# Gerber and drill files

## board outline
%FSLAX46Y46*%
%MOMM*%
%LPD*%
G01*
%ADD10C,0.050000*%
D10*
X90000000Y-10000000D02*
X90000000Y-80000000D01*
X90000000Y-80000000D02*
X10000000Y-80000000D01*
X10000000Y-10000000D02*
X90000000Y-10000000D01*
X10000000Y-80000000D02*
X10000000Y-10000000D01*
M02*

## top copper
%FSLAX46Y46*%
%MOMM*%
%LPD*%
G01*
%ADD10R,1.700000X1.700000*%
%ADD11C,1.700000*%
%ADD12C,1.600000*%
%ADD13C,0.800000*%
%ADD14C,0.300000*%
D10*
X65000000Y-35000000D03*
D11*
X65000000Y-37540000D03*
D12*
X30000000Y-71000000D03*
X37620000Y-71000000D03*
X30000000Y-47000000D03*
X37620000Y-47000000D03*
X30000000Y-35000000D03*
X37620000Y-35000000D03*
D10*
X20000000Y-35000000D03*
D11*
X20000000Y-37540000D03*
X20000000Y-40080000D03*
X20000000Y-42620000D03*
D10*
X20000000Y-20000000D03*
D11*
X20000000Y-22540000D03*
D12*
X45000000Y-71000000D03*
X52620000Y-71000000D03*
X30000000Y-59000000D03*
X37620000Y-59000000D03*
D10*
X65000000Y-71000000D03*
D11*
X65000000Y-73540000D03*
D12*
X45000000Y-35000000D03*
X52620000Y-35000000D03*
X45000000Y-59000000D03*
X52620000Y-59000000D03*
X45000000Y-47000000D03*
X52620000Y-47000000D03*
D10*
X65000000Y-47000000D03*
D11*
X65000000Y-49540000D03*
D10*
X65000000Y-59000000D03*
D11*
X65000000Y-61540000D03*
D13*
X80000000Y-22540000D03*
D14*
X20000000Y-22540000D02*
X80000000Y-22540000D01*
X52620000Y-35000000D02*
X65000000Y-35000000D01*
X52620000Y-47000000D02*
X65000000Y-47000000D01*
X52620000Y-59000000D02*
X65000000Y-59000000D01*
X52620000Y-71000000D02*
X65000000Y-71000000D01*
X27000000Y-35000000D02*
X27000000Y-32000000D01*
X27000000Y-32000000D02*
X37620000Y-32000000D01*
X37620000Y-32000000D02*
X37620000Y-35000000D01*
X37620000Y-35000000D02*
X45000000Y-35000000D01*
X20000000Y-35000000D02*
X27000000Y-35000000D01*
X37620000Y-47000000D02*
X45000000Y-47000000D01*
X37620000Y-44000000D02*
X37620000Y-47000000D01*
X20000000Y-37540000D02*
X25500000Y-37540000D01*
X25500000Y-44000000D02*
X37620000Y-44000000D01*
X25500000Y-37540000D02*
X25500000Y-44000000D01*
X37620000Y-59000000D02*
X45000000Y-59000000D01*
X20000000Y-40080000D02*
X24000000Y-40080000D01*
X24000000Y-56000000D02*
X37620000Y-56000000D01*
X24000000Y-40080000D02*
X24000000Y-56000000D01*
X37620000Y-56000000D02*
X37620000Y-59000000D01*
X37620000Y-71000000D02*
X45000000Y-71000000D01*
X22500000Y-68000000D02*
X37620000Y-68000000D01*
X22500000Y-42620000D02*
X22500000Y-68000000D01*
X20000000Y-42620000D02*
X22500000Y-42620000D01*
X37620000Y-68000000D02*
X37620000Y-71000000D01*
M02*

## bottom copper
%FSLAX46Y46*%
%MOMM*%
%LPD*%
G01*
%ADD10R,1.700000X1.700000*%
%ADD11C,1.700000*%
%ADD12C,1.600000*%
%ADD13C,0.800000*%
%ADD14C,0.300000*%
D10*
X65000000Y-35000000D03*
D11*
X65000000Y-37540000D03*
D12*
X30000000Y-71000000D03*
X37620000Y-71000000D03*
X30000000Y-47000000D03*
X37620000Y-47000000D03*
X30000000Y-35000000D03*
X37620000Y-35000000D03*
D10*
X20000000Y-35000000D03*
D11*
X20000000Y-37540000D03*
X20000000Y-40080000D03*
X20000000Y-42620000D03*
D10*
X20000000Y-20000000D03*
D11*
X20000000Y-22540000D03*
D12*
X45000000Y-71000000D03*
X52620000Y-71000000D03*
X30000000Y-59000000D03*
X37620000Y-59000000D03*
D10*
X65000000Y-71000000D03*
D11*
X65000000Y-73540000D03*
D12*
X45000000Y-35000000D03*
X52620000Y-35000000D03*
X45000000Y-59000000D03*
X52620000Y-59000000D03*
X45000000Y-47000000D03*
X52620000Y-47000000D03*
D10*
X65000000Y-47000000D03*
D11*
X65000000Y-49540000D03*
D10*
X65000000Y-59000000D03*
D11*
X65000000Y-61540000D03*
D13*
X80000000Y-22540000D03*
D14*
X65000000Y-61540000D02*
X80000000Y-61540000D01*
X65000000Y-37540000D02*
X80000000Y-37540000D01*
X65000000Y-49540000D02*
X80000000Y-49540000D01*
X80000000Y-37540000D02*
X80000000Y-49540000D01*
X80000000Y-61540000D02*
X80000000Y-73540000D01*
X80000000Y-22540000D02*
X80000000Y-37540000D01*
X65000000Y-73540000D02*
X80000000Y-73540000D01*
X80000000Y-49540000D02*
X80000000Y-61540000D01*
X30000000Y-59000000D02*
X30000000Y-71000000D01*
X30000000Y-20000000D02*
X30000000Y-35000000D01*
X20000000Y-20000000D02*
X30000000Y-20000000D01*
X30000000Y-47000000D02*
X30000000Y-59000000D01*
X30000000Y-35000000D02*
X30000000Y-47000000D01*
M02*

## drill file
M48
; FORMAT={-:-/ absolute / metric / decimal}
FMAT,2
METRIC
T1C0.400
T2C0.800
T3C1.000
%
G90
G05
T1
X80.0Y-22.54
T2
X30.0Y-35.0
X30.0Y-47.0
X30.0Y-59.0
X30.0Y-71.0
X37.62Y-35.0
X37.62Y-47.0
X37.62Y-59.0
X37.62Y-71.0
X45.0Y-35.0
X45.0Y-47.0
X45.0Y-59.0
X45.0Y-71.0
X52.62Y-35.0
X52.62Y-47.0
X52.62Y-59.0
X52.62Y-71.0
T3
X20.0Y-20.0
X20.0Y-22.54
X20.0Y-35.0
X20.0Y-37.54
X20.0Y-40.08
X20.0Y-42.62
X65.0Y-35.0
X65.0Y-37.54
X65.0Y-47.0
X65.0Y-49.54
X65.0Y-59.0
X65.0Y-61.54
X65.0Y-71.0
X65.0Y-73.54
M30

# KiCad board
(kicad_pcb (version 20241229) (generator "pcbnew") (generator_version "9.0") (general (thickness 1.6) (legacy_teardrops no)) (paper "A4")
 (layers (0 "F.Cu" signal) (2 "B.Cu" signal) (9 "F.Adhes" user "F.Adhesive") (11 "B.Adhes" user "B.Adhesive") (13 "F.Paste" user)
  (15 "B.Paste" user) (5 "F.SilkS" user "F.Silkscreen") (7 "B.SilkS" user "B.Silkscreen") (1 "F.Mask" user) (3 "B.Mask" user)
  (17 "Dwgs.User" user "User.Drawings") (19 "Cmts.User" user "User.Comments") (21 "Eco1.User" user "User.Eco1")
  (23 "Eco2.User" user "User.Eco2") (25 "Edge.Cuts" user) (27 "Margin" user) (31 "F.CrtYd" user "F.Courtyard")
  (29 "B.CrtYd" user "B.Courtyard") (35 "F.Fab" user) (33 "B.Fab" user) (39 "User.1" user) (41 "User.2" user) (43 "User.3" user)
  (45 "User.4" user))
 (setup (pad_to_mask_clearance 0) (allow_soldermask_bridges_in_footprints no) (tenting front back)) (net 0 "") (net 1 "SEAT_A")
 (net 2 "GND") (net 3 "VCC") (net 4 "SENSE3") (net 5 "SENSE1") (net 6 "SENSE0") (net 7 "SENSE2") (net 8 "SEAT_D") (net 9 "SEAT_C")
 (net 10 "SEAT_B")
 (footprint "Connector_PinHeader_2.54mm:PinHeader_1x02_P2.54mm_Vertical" (layer "F.Cu") (at 65 35)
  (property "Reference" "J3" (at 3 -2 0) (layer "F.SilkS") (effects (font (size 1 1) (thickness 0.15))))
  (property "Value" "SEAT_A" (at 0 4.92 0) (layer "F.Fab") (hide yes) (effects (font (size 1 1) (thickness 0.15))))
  (pad "1" thru_hole rect (at 0 0) (size 1.7 1.7) (drill 1) (layers "*.Cu" "*.Mask") (remove_unused_layers no) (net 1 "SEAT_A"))
  (pad "2" thru_hole circle (at 0 2.54) (size 1.7 1.7) (drill 1) (layers "*.Cu" "*.Mask") (remove_unused_layers no) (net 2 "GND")))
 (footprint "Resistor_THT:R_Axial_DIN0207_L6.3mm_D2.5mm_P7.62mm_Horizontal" (layer "F.Cu") (at 30 71)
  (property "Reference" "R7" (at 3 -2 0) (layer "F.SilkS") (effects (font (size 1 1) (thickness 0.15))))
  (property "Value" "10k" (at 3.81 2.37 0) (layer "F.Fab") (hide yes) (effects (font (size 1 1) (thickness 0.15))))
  (pad "1" thru_hole circle (at 0 0) (size 1.6 1.6) (drill 0.8) (layers "*.Cu" "*.Mask") (remove_unused_layers no) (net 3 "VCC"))
  (pad "2" thru_hole circle (at 7.62 0) (size 1.6 1.6) (drill 0.8) (layers "*.Cu" "*.Mask") (remove_unused_layers no) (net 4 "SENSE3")))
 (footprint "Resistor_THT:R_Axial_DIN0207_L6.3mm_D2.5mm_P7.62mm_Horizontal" (layer "F.Cu") (at 30 47)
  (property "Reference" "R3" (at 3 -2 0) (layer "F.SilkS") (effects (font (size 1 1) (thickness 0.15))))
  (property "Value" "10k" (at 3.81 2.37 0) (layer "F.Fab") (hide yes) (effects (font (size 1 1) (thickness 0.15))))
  (pad "1" thru_hole circle (at 0 0) (size 1.6 1.6) (drill 0.8) (layers "*.Cu" "*.Mask") (remove_unused_layers no) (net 3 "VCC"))
  (pad "2" thru_hole circle (at 7.62 0) (size 1.6 1.6) (drill 0.8) (layers "*.Cu" "*.Mask") (remove_unused_layers no) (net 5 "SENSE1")))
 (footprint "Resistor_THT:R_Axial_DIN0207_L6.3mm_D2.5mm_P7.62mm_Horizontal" (layer "F.Cu") (at 30 35)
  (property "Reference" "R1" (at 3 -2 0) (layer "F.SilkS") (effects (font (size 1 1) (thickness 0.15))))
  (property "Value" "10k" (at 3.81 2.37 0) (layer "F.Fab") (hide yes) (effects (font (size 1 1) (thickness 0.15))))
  (pad "1" thru_hole circle (at 0 0) (size 1.6 1.6) (drill 0.8) (layers "*.Cu" "*.Mask") (remove_unused_layers no) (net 3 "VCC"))
  (pad "2" thru_hole circle (at 7.62 0) (size 1.6 1.6) (drill 0.8) (layers "*.Cu" "*.Mask") (remove_unused_layers no) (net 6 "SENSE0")))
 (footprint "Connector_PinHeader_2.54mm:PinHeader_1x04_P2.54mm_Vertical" (layer "F.Cu") (at 20 35)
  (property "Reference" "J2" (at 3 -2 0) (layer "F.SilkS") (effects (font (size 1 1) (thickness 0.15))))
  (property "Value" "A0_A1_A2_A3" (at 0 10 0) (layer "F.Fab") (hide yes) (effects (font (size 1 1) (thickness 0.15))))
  (pad "1" thru_hole rect (at 0 0) (size 1.7 1.7) (drill 1) (layers "*.Cu" "*.Mask") (remove_unused_layers no) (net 6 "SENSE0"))
  (pad "2" thru_hole circle (at 0 2.54) (size 1.7 1.7) (drill 1) (layers "*.Cu" "*.Mask") (remove_unused_layers no) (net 5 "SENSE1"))
  (pad "3" thru_hole circle (at 0 5.08) (size 1.7 1.7) (drill 1) (layers "*.Cu" "*.Mask") (remove_unused_layers no) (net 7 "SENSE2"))
  (pad "4" thru_hole circle (at 0 7.62) (size 1.7 1.7) (drill 1) (layers "*.Cu" "*.Mask") (remove_unused_layers no) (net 4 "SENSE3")))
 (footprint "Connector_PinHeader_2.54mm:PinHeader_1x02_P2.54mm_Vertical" (layer "F.Cu") (at 20 20)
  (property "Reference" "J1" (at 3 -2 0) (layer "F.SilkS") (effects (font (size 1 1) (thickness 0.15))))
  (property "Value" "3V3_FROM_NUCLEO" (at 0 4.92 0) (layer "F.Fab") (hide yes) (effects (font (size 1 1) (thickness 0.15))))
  (pad "1" thru_hole rect (at 0 0) (size 1.7 1.7) (drill 1) (layers "*.Cu" "*.Mask") (remove_unused_layers no) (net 3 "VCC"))
  (pad "2" thru_hole circle (at 0 2.54) (size 1.7 1.7) (drill 1) (layers "*.Cu" "*.Mask") (remove_unused_layers no) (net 2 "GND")))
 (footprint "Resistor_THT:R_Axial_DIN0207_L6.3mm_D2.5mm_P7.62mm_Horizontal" (layer "F.Cu") (at 45 71)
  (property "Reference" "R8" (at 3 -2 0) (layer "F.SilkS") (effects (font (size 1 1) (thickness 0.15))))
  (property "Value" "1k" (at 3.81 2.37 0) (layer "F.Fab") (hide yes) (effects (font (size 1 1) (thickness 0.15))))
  (pad "1" thru_hole circle (at 0 0) (size 1.6 1.6) (drill 0.8) (layers "*.Cu" "*.Mask") (remove_unused_layers no) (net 4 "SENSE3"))
  (pad "2" thru_hole circle (at 7.62 0) (size 1.6 1.6) (drill 0.8) (layers "*.Cu" "*.Mask") (remove_unused_layers no) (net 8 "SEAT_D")))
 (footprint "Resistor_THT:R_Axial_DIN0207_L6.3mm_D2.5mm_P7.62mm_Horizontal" (layer "F.Cu") (at 30 59)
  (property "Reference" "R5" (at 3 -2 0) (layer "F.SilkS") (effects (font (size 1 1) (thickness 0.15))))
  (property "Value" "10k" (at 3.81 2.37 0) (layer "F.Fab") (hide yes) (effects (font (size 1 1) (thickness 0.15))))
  (pad "1" thru_hole circle (at 0 0) (size 1.6 1.6) (drill 0.8) (layers "*.Cu" "*.Mask") (remove_unused_layers no) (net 3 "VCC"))
  (pad "2" thru_hole circle (at 7.62 0) (size 1.6 1.6) (drill 0.8) (layers "*.Cu" "*.Mask") (remove_unused_layers no) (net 7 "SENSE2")))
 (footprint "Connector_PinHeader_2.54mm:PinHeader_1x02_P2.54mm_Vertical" (layer "F.Cu") (at 65 71)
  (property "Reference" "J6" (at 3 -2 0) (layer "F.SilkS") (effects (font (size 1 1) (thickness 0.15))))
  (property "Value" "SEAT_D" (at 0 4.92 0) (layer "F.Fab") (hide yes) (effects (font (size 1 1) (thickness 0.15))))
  (pad "1" thru_hole rect (at 0 0) (size 1.7 1.7) (drill 1) (layers "*.Cu" "*.Mask") (remove_unused_layers no) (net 8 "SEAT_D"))
  (pad "2" thru_hole circle (at 0 2.54) (size 1.7 1.7) (drill 1) (layers "*.Cu" "*.Mask") (remove_unused_layers no) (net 2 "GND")))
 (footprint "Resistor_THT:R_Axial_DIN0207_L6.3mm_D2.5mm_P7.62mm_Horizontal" (layer "F.Cu") (at 45 35)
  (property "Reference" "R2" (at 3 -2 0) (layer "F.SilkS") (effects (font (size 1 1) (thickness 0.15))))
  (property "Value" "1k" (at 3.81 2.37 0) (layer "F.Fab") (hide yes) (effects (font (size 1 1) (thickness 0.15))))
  (pad "1" thru_hole circle (at 0 0) (size 1.6 1.6) (drill 0.8) (layers "*.Cu" "*.Mask") (remove_unused_layers no) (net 6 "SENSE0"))
  (pad "2" thru_hole circle (at 7.62 0) (size 1.6 1.6) (drill 0.8) (layers "*.Cu" "*.Mask") (remove_unused_layers no) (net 1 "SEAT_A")))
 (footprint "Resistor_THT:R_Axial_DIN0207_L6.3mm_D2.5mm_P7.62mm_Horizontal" (layer "F.Cu") (at 45 59)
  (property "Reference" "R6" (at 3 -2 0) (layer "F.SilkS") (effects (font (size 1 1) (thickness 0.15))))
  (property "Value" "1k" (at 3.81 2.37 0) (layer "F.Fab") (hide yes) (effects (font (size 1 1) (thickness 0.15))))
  (pad "1" thru_hole circle (at 0 0) (size 1.6 1.6) (drill 0.8) (layers "*.Cu" "*.Mask") (remove_unused_layers no) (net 7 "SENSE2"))
  (pad "2" thru_hole circle (at 7.62 0) (size 1.6 1.6) (drill 0.8) (layers "*.Cu" "*.Mask") (remove_unused_layers no) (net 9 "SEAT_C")))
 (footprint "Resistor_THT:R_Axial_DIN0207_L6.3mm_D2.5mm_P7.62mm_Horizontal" (layer "F.Cu") (at 45 47)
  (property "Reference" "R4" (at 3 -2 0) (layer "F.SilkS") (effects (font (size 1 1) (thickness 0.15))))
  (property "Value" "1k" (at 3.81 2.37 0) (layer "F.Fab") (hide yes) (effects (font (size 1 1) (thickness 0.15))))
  (pad "1" thru_hole circle (at 0 0) (size 1.6 1.6) (drill 0.8) (layers "*.Cu" "*.Mask") (remove_unused_layers no) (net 5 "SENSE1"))
  (pad "2" thru_hole circle (at 7.62 0) (size 1.6 1.6) (drill 0.8) (layers "*.Cu" "*.Mask") (remove_unused_layers no) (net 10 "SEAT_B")))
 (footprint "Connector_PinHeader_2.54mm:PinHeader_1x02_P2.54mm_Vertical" (layer "F.Cu") (at 65 47)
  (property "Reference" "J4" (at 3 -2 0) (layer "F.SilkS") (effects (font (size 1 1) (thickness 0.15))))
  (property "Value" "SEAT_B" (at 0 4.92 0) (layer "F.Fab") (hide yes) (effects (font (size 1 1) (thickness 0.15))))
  (pad "1" thru_hole rect (at 0 0) (size 1.7 1.7) (drill 1) (layers "*.Cu" "*.Mask") (remove_unused_layers no) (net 10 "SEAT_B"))
  (pad "2" thru_hole circle (at 0 2.54) (size 1.7 1.7) (drill 1) (layers "*.Cu" "*.Mask") (remove_unused_layers no) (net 2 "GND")))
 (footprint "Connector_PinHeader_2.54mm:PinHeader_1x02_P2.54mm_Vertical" (layer "F.Cu") (at 65 59)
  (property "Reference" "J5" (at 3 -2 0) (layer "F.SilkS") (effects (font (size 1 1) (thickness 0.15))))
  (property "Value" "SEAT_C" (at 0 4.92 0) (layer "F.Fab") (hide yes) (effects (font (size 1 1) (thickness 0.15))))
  (pad "1" thru_hole rect (at 0 0) (size 1.7 1.7) (drill 1) (layers "*.Cu" "*.Mask") (remove_unused_layers no) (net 9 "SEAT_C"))
  (pad "2" thru_hole circle (at 0 2.54) (size 1.7 1.7) (drill 1) (layers "*.Cu" "*.Mask") (remove_unused_layers no) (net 2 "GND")))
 (gr_line (start 90 10) (end 90 80) (stroke (width 0.05) (type default)) (layer "Edge.Cuts"))
 (gr_line (start 90 80) (end 10 80) (stroke (width 0.05) (type default)) (layer "Edge.Cuts"))
 (gr_line (start 10 10) (end 90 10) (stroke (width 0.05) (type default)) (layer "Edge.Cuts"))
 (gr_line (start 10 80) (end 10 10) (stroke (width 0.05) (type default)) (layer "Edge.Cuts"))
 (segment (start 20 22.54) (end 80 22.54) (width 0.3) (layer "F.Cu") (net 2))
 (via (at 80 22.54) (size 0.8) (drill 0.4) (layers "F.Cu" "B.Cu") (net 2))
 (segment (start 65 61.54) (end 80 61.54) (width 0.3) (layer "B.Cu") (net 2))
 (segment (start 65 37.54) (end 80 37.54) (width 0.3) (layer "B.Cu") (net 2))
 (segment (start 65 49.54) (end 80 49.54) (width 0.3) (layer "B.Cu") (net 2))
 (segment (start 80 37.54) (end 80 49.54) (width 0.3) (layer "B.Cu") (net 2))
 (segment (start 80 61.54) (end 80 73.54) (width 0.3) (layer "B.Cu") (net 2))
 (segment (start 80 22.54) (end 80 37.54) (width 0.3) (layer "B.Cu") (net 2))
 (segment (start 65 73.54) (end 80 73.54) (width 0.3) (layer "B.Cu") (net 2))
 (segment (start 80 49.54) (end 80 61.54) (width 0.3) (layer "B.Cu") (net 2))
 (segment (start 52.62 35) (end 65 35) (width 0.3) (layer "F.Cu") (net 1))
 (segment (start 52.62 47) (end 65 47) (width 0.3) (layer "F.Cu") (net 10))
 (segment (start 52.62 59) (end 65 59) (width 0.3) (layer "F.Cu") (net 9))
 (segment (start 52.62 71) (end 65 71) (width 0.3) (layer "F.Cu") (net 8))
 (segment (start 27 35) (end 27 32) (width 0.3) (layer "F.Cu") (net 6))
 (segment (start 27 32) (end 37.62 32) (width 0.3) (layer "F.Cu") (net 6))
 (segment (start 37.62 32) (end 37.62 35) (width 0.3) (layer "F.Cu") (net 6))
 (segment (start 37.62 35) (end 45 35) (width 0.3) (layer "F.Cu") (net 6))
 (segment (start 20 35) (end 27 35) (width 0.3) (layer "F.Cu") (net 6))
 (segment (start 37.62 47) (end 45 47) (width 0.3) (layer "F.Cu") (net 5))
 (segment (start 37.62 44) (end 37.62 47) (width 0.3) (layer "F.Cu") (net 5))
 (segment (start 20 37.54) (end 25.5 37.54) (width 0.3) (layer "F.Cu") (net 5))
 (segment (start 25.5 44) (end 37.62 44) (width 0.3) (layer "F.Cu") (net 5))
 (segment (start 25.5 37.54) (end 25.5 44) (width 0.3) (layer "F.Cu") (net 5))
 (segment (start 37.62 59) (end 45 59) (width 0.3) (layer "F.Cu") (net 7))
 (segment (start 20 40.08) (end 24 40.08) (width 0.3) (layer "F.Cu") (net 7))
 (segment (start 24 56) (end 37.62 56) (width 0.3) (layer "F.Cu") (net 7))
 (segment (start 24 40.08) (end 24 56) (width 0.3) (layer "F.Cu") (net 7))
 (segment (start 37.62 56) (end 37.62 59) (width 0.3) (layer "F.Cu") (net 7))
 (segment (start 37.62 71) (end 45 71) (width 0.3) (layer "F.Cu") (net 4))
 (segment (start 22.5 68) (end 37.62 68) (width 0.3) (layer "F.Cu") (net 4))
 (segment (start 22.5 42.62) (end 22.5 68) (width 0.3) (layer "F.Cu") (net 4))
 (segment (start 20 42.62) (end 22.5 42.62) (width 0.3) (layer "F.Cu") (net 4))
 (segment (start 37.62 68) (end 37.62 71) (width 0.3) (layer "F.Cu") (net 4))
 (segment (start 30 59) (end 30 71) (width 0.3) (layer "B.Cu") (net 3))
 (segment (start 30 20) (end 30 35) (width 0.3) (layer "B.Cu") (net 3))
 (segment (start 20 20) (end 30 20) (width 0.3) (layer "B.Cu") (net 3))
 (segment (start 30 47) (end 30 59) (width 0.3) (layer "B.Cu") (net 3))
 (segment (start 30 35) (end 30 47) (width 0.3) (layer "B.Cu") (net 3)))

